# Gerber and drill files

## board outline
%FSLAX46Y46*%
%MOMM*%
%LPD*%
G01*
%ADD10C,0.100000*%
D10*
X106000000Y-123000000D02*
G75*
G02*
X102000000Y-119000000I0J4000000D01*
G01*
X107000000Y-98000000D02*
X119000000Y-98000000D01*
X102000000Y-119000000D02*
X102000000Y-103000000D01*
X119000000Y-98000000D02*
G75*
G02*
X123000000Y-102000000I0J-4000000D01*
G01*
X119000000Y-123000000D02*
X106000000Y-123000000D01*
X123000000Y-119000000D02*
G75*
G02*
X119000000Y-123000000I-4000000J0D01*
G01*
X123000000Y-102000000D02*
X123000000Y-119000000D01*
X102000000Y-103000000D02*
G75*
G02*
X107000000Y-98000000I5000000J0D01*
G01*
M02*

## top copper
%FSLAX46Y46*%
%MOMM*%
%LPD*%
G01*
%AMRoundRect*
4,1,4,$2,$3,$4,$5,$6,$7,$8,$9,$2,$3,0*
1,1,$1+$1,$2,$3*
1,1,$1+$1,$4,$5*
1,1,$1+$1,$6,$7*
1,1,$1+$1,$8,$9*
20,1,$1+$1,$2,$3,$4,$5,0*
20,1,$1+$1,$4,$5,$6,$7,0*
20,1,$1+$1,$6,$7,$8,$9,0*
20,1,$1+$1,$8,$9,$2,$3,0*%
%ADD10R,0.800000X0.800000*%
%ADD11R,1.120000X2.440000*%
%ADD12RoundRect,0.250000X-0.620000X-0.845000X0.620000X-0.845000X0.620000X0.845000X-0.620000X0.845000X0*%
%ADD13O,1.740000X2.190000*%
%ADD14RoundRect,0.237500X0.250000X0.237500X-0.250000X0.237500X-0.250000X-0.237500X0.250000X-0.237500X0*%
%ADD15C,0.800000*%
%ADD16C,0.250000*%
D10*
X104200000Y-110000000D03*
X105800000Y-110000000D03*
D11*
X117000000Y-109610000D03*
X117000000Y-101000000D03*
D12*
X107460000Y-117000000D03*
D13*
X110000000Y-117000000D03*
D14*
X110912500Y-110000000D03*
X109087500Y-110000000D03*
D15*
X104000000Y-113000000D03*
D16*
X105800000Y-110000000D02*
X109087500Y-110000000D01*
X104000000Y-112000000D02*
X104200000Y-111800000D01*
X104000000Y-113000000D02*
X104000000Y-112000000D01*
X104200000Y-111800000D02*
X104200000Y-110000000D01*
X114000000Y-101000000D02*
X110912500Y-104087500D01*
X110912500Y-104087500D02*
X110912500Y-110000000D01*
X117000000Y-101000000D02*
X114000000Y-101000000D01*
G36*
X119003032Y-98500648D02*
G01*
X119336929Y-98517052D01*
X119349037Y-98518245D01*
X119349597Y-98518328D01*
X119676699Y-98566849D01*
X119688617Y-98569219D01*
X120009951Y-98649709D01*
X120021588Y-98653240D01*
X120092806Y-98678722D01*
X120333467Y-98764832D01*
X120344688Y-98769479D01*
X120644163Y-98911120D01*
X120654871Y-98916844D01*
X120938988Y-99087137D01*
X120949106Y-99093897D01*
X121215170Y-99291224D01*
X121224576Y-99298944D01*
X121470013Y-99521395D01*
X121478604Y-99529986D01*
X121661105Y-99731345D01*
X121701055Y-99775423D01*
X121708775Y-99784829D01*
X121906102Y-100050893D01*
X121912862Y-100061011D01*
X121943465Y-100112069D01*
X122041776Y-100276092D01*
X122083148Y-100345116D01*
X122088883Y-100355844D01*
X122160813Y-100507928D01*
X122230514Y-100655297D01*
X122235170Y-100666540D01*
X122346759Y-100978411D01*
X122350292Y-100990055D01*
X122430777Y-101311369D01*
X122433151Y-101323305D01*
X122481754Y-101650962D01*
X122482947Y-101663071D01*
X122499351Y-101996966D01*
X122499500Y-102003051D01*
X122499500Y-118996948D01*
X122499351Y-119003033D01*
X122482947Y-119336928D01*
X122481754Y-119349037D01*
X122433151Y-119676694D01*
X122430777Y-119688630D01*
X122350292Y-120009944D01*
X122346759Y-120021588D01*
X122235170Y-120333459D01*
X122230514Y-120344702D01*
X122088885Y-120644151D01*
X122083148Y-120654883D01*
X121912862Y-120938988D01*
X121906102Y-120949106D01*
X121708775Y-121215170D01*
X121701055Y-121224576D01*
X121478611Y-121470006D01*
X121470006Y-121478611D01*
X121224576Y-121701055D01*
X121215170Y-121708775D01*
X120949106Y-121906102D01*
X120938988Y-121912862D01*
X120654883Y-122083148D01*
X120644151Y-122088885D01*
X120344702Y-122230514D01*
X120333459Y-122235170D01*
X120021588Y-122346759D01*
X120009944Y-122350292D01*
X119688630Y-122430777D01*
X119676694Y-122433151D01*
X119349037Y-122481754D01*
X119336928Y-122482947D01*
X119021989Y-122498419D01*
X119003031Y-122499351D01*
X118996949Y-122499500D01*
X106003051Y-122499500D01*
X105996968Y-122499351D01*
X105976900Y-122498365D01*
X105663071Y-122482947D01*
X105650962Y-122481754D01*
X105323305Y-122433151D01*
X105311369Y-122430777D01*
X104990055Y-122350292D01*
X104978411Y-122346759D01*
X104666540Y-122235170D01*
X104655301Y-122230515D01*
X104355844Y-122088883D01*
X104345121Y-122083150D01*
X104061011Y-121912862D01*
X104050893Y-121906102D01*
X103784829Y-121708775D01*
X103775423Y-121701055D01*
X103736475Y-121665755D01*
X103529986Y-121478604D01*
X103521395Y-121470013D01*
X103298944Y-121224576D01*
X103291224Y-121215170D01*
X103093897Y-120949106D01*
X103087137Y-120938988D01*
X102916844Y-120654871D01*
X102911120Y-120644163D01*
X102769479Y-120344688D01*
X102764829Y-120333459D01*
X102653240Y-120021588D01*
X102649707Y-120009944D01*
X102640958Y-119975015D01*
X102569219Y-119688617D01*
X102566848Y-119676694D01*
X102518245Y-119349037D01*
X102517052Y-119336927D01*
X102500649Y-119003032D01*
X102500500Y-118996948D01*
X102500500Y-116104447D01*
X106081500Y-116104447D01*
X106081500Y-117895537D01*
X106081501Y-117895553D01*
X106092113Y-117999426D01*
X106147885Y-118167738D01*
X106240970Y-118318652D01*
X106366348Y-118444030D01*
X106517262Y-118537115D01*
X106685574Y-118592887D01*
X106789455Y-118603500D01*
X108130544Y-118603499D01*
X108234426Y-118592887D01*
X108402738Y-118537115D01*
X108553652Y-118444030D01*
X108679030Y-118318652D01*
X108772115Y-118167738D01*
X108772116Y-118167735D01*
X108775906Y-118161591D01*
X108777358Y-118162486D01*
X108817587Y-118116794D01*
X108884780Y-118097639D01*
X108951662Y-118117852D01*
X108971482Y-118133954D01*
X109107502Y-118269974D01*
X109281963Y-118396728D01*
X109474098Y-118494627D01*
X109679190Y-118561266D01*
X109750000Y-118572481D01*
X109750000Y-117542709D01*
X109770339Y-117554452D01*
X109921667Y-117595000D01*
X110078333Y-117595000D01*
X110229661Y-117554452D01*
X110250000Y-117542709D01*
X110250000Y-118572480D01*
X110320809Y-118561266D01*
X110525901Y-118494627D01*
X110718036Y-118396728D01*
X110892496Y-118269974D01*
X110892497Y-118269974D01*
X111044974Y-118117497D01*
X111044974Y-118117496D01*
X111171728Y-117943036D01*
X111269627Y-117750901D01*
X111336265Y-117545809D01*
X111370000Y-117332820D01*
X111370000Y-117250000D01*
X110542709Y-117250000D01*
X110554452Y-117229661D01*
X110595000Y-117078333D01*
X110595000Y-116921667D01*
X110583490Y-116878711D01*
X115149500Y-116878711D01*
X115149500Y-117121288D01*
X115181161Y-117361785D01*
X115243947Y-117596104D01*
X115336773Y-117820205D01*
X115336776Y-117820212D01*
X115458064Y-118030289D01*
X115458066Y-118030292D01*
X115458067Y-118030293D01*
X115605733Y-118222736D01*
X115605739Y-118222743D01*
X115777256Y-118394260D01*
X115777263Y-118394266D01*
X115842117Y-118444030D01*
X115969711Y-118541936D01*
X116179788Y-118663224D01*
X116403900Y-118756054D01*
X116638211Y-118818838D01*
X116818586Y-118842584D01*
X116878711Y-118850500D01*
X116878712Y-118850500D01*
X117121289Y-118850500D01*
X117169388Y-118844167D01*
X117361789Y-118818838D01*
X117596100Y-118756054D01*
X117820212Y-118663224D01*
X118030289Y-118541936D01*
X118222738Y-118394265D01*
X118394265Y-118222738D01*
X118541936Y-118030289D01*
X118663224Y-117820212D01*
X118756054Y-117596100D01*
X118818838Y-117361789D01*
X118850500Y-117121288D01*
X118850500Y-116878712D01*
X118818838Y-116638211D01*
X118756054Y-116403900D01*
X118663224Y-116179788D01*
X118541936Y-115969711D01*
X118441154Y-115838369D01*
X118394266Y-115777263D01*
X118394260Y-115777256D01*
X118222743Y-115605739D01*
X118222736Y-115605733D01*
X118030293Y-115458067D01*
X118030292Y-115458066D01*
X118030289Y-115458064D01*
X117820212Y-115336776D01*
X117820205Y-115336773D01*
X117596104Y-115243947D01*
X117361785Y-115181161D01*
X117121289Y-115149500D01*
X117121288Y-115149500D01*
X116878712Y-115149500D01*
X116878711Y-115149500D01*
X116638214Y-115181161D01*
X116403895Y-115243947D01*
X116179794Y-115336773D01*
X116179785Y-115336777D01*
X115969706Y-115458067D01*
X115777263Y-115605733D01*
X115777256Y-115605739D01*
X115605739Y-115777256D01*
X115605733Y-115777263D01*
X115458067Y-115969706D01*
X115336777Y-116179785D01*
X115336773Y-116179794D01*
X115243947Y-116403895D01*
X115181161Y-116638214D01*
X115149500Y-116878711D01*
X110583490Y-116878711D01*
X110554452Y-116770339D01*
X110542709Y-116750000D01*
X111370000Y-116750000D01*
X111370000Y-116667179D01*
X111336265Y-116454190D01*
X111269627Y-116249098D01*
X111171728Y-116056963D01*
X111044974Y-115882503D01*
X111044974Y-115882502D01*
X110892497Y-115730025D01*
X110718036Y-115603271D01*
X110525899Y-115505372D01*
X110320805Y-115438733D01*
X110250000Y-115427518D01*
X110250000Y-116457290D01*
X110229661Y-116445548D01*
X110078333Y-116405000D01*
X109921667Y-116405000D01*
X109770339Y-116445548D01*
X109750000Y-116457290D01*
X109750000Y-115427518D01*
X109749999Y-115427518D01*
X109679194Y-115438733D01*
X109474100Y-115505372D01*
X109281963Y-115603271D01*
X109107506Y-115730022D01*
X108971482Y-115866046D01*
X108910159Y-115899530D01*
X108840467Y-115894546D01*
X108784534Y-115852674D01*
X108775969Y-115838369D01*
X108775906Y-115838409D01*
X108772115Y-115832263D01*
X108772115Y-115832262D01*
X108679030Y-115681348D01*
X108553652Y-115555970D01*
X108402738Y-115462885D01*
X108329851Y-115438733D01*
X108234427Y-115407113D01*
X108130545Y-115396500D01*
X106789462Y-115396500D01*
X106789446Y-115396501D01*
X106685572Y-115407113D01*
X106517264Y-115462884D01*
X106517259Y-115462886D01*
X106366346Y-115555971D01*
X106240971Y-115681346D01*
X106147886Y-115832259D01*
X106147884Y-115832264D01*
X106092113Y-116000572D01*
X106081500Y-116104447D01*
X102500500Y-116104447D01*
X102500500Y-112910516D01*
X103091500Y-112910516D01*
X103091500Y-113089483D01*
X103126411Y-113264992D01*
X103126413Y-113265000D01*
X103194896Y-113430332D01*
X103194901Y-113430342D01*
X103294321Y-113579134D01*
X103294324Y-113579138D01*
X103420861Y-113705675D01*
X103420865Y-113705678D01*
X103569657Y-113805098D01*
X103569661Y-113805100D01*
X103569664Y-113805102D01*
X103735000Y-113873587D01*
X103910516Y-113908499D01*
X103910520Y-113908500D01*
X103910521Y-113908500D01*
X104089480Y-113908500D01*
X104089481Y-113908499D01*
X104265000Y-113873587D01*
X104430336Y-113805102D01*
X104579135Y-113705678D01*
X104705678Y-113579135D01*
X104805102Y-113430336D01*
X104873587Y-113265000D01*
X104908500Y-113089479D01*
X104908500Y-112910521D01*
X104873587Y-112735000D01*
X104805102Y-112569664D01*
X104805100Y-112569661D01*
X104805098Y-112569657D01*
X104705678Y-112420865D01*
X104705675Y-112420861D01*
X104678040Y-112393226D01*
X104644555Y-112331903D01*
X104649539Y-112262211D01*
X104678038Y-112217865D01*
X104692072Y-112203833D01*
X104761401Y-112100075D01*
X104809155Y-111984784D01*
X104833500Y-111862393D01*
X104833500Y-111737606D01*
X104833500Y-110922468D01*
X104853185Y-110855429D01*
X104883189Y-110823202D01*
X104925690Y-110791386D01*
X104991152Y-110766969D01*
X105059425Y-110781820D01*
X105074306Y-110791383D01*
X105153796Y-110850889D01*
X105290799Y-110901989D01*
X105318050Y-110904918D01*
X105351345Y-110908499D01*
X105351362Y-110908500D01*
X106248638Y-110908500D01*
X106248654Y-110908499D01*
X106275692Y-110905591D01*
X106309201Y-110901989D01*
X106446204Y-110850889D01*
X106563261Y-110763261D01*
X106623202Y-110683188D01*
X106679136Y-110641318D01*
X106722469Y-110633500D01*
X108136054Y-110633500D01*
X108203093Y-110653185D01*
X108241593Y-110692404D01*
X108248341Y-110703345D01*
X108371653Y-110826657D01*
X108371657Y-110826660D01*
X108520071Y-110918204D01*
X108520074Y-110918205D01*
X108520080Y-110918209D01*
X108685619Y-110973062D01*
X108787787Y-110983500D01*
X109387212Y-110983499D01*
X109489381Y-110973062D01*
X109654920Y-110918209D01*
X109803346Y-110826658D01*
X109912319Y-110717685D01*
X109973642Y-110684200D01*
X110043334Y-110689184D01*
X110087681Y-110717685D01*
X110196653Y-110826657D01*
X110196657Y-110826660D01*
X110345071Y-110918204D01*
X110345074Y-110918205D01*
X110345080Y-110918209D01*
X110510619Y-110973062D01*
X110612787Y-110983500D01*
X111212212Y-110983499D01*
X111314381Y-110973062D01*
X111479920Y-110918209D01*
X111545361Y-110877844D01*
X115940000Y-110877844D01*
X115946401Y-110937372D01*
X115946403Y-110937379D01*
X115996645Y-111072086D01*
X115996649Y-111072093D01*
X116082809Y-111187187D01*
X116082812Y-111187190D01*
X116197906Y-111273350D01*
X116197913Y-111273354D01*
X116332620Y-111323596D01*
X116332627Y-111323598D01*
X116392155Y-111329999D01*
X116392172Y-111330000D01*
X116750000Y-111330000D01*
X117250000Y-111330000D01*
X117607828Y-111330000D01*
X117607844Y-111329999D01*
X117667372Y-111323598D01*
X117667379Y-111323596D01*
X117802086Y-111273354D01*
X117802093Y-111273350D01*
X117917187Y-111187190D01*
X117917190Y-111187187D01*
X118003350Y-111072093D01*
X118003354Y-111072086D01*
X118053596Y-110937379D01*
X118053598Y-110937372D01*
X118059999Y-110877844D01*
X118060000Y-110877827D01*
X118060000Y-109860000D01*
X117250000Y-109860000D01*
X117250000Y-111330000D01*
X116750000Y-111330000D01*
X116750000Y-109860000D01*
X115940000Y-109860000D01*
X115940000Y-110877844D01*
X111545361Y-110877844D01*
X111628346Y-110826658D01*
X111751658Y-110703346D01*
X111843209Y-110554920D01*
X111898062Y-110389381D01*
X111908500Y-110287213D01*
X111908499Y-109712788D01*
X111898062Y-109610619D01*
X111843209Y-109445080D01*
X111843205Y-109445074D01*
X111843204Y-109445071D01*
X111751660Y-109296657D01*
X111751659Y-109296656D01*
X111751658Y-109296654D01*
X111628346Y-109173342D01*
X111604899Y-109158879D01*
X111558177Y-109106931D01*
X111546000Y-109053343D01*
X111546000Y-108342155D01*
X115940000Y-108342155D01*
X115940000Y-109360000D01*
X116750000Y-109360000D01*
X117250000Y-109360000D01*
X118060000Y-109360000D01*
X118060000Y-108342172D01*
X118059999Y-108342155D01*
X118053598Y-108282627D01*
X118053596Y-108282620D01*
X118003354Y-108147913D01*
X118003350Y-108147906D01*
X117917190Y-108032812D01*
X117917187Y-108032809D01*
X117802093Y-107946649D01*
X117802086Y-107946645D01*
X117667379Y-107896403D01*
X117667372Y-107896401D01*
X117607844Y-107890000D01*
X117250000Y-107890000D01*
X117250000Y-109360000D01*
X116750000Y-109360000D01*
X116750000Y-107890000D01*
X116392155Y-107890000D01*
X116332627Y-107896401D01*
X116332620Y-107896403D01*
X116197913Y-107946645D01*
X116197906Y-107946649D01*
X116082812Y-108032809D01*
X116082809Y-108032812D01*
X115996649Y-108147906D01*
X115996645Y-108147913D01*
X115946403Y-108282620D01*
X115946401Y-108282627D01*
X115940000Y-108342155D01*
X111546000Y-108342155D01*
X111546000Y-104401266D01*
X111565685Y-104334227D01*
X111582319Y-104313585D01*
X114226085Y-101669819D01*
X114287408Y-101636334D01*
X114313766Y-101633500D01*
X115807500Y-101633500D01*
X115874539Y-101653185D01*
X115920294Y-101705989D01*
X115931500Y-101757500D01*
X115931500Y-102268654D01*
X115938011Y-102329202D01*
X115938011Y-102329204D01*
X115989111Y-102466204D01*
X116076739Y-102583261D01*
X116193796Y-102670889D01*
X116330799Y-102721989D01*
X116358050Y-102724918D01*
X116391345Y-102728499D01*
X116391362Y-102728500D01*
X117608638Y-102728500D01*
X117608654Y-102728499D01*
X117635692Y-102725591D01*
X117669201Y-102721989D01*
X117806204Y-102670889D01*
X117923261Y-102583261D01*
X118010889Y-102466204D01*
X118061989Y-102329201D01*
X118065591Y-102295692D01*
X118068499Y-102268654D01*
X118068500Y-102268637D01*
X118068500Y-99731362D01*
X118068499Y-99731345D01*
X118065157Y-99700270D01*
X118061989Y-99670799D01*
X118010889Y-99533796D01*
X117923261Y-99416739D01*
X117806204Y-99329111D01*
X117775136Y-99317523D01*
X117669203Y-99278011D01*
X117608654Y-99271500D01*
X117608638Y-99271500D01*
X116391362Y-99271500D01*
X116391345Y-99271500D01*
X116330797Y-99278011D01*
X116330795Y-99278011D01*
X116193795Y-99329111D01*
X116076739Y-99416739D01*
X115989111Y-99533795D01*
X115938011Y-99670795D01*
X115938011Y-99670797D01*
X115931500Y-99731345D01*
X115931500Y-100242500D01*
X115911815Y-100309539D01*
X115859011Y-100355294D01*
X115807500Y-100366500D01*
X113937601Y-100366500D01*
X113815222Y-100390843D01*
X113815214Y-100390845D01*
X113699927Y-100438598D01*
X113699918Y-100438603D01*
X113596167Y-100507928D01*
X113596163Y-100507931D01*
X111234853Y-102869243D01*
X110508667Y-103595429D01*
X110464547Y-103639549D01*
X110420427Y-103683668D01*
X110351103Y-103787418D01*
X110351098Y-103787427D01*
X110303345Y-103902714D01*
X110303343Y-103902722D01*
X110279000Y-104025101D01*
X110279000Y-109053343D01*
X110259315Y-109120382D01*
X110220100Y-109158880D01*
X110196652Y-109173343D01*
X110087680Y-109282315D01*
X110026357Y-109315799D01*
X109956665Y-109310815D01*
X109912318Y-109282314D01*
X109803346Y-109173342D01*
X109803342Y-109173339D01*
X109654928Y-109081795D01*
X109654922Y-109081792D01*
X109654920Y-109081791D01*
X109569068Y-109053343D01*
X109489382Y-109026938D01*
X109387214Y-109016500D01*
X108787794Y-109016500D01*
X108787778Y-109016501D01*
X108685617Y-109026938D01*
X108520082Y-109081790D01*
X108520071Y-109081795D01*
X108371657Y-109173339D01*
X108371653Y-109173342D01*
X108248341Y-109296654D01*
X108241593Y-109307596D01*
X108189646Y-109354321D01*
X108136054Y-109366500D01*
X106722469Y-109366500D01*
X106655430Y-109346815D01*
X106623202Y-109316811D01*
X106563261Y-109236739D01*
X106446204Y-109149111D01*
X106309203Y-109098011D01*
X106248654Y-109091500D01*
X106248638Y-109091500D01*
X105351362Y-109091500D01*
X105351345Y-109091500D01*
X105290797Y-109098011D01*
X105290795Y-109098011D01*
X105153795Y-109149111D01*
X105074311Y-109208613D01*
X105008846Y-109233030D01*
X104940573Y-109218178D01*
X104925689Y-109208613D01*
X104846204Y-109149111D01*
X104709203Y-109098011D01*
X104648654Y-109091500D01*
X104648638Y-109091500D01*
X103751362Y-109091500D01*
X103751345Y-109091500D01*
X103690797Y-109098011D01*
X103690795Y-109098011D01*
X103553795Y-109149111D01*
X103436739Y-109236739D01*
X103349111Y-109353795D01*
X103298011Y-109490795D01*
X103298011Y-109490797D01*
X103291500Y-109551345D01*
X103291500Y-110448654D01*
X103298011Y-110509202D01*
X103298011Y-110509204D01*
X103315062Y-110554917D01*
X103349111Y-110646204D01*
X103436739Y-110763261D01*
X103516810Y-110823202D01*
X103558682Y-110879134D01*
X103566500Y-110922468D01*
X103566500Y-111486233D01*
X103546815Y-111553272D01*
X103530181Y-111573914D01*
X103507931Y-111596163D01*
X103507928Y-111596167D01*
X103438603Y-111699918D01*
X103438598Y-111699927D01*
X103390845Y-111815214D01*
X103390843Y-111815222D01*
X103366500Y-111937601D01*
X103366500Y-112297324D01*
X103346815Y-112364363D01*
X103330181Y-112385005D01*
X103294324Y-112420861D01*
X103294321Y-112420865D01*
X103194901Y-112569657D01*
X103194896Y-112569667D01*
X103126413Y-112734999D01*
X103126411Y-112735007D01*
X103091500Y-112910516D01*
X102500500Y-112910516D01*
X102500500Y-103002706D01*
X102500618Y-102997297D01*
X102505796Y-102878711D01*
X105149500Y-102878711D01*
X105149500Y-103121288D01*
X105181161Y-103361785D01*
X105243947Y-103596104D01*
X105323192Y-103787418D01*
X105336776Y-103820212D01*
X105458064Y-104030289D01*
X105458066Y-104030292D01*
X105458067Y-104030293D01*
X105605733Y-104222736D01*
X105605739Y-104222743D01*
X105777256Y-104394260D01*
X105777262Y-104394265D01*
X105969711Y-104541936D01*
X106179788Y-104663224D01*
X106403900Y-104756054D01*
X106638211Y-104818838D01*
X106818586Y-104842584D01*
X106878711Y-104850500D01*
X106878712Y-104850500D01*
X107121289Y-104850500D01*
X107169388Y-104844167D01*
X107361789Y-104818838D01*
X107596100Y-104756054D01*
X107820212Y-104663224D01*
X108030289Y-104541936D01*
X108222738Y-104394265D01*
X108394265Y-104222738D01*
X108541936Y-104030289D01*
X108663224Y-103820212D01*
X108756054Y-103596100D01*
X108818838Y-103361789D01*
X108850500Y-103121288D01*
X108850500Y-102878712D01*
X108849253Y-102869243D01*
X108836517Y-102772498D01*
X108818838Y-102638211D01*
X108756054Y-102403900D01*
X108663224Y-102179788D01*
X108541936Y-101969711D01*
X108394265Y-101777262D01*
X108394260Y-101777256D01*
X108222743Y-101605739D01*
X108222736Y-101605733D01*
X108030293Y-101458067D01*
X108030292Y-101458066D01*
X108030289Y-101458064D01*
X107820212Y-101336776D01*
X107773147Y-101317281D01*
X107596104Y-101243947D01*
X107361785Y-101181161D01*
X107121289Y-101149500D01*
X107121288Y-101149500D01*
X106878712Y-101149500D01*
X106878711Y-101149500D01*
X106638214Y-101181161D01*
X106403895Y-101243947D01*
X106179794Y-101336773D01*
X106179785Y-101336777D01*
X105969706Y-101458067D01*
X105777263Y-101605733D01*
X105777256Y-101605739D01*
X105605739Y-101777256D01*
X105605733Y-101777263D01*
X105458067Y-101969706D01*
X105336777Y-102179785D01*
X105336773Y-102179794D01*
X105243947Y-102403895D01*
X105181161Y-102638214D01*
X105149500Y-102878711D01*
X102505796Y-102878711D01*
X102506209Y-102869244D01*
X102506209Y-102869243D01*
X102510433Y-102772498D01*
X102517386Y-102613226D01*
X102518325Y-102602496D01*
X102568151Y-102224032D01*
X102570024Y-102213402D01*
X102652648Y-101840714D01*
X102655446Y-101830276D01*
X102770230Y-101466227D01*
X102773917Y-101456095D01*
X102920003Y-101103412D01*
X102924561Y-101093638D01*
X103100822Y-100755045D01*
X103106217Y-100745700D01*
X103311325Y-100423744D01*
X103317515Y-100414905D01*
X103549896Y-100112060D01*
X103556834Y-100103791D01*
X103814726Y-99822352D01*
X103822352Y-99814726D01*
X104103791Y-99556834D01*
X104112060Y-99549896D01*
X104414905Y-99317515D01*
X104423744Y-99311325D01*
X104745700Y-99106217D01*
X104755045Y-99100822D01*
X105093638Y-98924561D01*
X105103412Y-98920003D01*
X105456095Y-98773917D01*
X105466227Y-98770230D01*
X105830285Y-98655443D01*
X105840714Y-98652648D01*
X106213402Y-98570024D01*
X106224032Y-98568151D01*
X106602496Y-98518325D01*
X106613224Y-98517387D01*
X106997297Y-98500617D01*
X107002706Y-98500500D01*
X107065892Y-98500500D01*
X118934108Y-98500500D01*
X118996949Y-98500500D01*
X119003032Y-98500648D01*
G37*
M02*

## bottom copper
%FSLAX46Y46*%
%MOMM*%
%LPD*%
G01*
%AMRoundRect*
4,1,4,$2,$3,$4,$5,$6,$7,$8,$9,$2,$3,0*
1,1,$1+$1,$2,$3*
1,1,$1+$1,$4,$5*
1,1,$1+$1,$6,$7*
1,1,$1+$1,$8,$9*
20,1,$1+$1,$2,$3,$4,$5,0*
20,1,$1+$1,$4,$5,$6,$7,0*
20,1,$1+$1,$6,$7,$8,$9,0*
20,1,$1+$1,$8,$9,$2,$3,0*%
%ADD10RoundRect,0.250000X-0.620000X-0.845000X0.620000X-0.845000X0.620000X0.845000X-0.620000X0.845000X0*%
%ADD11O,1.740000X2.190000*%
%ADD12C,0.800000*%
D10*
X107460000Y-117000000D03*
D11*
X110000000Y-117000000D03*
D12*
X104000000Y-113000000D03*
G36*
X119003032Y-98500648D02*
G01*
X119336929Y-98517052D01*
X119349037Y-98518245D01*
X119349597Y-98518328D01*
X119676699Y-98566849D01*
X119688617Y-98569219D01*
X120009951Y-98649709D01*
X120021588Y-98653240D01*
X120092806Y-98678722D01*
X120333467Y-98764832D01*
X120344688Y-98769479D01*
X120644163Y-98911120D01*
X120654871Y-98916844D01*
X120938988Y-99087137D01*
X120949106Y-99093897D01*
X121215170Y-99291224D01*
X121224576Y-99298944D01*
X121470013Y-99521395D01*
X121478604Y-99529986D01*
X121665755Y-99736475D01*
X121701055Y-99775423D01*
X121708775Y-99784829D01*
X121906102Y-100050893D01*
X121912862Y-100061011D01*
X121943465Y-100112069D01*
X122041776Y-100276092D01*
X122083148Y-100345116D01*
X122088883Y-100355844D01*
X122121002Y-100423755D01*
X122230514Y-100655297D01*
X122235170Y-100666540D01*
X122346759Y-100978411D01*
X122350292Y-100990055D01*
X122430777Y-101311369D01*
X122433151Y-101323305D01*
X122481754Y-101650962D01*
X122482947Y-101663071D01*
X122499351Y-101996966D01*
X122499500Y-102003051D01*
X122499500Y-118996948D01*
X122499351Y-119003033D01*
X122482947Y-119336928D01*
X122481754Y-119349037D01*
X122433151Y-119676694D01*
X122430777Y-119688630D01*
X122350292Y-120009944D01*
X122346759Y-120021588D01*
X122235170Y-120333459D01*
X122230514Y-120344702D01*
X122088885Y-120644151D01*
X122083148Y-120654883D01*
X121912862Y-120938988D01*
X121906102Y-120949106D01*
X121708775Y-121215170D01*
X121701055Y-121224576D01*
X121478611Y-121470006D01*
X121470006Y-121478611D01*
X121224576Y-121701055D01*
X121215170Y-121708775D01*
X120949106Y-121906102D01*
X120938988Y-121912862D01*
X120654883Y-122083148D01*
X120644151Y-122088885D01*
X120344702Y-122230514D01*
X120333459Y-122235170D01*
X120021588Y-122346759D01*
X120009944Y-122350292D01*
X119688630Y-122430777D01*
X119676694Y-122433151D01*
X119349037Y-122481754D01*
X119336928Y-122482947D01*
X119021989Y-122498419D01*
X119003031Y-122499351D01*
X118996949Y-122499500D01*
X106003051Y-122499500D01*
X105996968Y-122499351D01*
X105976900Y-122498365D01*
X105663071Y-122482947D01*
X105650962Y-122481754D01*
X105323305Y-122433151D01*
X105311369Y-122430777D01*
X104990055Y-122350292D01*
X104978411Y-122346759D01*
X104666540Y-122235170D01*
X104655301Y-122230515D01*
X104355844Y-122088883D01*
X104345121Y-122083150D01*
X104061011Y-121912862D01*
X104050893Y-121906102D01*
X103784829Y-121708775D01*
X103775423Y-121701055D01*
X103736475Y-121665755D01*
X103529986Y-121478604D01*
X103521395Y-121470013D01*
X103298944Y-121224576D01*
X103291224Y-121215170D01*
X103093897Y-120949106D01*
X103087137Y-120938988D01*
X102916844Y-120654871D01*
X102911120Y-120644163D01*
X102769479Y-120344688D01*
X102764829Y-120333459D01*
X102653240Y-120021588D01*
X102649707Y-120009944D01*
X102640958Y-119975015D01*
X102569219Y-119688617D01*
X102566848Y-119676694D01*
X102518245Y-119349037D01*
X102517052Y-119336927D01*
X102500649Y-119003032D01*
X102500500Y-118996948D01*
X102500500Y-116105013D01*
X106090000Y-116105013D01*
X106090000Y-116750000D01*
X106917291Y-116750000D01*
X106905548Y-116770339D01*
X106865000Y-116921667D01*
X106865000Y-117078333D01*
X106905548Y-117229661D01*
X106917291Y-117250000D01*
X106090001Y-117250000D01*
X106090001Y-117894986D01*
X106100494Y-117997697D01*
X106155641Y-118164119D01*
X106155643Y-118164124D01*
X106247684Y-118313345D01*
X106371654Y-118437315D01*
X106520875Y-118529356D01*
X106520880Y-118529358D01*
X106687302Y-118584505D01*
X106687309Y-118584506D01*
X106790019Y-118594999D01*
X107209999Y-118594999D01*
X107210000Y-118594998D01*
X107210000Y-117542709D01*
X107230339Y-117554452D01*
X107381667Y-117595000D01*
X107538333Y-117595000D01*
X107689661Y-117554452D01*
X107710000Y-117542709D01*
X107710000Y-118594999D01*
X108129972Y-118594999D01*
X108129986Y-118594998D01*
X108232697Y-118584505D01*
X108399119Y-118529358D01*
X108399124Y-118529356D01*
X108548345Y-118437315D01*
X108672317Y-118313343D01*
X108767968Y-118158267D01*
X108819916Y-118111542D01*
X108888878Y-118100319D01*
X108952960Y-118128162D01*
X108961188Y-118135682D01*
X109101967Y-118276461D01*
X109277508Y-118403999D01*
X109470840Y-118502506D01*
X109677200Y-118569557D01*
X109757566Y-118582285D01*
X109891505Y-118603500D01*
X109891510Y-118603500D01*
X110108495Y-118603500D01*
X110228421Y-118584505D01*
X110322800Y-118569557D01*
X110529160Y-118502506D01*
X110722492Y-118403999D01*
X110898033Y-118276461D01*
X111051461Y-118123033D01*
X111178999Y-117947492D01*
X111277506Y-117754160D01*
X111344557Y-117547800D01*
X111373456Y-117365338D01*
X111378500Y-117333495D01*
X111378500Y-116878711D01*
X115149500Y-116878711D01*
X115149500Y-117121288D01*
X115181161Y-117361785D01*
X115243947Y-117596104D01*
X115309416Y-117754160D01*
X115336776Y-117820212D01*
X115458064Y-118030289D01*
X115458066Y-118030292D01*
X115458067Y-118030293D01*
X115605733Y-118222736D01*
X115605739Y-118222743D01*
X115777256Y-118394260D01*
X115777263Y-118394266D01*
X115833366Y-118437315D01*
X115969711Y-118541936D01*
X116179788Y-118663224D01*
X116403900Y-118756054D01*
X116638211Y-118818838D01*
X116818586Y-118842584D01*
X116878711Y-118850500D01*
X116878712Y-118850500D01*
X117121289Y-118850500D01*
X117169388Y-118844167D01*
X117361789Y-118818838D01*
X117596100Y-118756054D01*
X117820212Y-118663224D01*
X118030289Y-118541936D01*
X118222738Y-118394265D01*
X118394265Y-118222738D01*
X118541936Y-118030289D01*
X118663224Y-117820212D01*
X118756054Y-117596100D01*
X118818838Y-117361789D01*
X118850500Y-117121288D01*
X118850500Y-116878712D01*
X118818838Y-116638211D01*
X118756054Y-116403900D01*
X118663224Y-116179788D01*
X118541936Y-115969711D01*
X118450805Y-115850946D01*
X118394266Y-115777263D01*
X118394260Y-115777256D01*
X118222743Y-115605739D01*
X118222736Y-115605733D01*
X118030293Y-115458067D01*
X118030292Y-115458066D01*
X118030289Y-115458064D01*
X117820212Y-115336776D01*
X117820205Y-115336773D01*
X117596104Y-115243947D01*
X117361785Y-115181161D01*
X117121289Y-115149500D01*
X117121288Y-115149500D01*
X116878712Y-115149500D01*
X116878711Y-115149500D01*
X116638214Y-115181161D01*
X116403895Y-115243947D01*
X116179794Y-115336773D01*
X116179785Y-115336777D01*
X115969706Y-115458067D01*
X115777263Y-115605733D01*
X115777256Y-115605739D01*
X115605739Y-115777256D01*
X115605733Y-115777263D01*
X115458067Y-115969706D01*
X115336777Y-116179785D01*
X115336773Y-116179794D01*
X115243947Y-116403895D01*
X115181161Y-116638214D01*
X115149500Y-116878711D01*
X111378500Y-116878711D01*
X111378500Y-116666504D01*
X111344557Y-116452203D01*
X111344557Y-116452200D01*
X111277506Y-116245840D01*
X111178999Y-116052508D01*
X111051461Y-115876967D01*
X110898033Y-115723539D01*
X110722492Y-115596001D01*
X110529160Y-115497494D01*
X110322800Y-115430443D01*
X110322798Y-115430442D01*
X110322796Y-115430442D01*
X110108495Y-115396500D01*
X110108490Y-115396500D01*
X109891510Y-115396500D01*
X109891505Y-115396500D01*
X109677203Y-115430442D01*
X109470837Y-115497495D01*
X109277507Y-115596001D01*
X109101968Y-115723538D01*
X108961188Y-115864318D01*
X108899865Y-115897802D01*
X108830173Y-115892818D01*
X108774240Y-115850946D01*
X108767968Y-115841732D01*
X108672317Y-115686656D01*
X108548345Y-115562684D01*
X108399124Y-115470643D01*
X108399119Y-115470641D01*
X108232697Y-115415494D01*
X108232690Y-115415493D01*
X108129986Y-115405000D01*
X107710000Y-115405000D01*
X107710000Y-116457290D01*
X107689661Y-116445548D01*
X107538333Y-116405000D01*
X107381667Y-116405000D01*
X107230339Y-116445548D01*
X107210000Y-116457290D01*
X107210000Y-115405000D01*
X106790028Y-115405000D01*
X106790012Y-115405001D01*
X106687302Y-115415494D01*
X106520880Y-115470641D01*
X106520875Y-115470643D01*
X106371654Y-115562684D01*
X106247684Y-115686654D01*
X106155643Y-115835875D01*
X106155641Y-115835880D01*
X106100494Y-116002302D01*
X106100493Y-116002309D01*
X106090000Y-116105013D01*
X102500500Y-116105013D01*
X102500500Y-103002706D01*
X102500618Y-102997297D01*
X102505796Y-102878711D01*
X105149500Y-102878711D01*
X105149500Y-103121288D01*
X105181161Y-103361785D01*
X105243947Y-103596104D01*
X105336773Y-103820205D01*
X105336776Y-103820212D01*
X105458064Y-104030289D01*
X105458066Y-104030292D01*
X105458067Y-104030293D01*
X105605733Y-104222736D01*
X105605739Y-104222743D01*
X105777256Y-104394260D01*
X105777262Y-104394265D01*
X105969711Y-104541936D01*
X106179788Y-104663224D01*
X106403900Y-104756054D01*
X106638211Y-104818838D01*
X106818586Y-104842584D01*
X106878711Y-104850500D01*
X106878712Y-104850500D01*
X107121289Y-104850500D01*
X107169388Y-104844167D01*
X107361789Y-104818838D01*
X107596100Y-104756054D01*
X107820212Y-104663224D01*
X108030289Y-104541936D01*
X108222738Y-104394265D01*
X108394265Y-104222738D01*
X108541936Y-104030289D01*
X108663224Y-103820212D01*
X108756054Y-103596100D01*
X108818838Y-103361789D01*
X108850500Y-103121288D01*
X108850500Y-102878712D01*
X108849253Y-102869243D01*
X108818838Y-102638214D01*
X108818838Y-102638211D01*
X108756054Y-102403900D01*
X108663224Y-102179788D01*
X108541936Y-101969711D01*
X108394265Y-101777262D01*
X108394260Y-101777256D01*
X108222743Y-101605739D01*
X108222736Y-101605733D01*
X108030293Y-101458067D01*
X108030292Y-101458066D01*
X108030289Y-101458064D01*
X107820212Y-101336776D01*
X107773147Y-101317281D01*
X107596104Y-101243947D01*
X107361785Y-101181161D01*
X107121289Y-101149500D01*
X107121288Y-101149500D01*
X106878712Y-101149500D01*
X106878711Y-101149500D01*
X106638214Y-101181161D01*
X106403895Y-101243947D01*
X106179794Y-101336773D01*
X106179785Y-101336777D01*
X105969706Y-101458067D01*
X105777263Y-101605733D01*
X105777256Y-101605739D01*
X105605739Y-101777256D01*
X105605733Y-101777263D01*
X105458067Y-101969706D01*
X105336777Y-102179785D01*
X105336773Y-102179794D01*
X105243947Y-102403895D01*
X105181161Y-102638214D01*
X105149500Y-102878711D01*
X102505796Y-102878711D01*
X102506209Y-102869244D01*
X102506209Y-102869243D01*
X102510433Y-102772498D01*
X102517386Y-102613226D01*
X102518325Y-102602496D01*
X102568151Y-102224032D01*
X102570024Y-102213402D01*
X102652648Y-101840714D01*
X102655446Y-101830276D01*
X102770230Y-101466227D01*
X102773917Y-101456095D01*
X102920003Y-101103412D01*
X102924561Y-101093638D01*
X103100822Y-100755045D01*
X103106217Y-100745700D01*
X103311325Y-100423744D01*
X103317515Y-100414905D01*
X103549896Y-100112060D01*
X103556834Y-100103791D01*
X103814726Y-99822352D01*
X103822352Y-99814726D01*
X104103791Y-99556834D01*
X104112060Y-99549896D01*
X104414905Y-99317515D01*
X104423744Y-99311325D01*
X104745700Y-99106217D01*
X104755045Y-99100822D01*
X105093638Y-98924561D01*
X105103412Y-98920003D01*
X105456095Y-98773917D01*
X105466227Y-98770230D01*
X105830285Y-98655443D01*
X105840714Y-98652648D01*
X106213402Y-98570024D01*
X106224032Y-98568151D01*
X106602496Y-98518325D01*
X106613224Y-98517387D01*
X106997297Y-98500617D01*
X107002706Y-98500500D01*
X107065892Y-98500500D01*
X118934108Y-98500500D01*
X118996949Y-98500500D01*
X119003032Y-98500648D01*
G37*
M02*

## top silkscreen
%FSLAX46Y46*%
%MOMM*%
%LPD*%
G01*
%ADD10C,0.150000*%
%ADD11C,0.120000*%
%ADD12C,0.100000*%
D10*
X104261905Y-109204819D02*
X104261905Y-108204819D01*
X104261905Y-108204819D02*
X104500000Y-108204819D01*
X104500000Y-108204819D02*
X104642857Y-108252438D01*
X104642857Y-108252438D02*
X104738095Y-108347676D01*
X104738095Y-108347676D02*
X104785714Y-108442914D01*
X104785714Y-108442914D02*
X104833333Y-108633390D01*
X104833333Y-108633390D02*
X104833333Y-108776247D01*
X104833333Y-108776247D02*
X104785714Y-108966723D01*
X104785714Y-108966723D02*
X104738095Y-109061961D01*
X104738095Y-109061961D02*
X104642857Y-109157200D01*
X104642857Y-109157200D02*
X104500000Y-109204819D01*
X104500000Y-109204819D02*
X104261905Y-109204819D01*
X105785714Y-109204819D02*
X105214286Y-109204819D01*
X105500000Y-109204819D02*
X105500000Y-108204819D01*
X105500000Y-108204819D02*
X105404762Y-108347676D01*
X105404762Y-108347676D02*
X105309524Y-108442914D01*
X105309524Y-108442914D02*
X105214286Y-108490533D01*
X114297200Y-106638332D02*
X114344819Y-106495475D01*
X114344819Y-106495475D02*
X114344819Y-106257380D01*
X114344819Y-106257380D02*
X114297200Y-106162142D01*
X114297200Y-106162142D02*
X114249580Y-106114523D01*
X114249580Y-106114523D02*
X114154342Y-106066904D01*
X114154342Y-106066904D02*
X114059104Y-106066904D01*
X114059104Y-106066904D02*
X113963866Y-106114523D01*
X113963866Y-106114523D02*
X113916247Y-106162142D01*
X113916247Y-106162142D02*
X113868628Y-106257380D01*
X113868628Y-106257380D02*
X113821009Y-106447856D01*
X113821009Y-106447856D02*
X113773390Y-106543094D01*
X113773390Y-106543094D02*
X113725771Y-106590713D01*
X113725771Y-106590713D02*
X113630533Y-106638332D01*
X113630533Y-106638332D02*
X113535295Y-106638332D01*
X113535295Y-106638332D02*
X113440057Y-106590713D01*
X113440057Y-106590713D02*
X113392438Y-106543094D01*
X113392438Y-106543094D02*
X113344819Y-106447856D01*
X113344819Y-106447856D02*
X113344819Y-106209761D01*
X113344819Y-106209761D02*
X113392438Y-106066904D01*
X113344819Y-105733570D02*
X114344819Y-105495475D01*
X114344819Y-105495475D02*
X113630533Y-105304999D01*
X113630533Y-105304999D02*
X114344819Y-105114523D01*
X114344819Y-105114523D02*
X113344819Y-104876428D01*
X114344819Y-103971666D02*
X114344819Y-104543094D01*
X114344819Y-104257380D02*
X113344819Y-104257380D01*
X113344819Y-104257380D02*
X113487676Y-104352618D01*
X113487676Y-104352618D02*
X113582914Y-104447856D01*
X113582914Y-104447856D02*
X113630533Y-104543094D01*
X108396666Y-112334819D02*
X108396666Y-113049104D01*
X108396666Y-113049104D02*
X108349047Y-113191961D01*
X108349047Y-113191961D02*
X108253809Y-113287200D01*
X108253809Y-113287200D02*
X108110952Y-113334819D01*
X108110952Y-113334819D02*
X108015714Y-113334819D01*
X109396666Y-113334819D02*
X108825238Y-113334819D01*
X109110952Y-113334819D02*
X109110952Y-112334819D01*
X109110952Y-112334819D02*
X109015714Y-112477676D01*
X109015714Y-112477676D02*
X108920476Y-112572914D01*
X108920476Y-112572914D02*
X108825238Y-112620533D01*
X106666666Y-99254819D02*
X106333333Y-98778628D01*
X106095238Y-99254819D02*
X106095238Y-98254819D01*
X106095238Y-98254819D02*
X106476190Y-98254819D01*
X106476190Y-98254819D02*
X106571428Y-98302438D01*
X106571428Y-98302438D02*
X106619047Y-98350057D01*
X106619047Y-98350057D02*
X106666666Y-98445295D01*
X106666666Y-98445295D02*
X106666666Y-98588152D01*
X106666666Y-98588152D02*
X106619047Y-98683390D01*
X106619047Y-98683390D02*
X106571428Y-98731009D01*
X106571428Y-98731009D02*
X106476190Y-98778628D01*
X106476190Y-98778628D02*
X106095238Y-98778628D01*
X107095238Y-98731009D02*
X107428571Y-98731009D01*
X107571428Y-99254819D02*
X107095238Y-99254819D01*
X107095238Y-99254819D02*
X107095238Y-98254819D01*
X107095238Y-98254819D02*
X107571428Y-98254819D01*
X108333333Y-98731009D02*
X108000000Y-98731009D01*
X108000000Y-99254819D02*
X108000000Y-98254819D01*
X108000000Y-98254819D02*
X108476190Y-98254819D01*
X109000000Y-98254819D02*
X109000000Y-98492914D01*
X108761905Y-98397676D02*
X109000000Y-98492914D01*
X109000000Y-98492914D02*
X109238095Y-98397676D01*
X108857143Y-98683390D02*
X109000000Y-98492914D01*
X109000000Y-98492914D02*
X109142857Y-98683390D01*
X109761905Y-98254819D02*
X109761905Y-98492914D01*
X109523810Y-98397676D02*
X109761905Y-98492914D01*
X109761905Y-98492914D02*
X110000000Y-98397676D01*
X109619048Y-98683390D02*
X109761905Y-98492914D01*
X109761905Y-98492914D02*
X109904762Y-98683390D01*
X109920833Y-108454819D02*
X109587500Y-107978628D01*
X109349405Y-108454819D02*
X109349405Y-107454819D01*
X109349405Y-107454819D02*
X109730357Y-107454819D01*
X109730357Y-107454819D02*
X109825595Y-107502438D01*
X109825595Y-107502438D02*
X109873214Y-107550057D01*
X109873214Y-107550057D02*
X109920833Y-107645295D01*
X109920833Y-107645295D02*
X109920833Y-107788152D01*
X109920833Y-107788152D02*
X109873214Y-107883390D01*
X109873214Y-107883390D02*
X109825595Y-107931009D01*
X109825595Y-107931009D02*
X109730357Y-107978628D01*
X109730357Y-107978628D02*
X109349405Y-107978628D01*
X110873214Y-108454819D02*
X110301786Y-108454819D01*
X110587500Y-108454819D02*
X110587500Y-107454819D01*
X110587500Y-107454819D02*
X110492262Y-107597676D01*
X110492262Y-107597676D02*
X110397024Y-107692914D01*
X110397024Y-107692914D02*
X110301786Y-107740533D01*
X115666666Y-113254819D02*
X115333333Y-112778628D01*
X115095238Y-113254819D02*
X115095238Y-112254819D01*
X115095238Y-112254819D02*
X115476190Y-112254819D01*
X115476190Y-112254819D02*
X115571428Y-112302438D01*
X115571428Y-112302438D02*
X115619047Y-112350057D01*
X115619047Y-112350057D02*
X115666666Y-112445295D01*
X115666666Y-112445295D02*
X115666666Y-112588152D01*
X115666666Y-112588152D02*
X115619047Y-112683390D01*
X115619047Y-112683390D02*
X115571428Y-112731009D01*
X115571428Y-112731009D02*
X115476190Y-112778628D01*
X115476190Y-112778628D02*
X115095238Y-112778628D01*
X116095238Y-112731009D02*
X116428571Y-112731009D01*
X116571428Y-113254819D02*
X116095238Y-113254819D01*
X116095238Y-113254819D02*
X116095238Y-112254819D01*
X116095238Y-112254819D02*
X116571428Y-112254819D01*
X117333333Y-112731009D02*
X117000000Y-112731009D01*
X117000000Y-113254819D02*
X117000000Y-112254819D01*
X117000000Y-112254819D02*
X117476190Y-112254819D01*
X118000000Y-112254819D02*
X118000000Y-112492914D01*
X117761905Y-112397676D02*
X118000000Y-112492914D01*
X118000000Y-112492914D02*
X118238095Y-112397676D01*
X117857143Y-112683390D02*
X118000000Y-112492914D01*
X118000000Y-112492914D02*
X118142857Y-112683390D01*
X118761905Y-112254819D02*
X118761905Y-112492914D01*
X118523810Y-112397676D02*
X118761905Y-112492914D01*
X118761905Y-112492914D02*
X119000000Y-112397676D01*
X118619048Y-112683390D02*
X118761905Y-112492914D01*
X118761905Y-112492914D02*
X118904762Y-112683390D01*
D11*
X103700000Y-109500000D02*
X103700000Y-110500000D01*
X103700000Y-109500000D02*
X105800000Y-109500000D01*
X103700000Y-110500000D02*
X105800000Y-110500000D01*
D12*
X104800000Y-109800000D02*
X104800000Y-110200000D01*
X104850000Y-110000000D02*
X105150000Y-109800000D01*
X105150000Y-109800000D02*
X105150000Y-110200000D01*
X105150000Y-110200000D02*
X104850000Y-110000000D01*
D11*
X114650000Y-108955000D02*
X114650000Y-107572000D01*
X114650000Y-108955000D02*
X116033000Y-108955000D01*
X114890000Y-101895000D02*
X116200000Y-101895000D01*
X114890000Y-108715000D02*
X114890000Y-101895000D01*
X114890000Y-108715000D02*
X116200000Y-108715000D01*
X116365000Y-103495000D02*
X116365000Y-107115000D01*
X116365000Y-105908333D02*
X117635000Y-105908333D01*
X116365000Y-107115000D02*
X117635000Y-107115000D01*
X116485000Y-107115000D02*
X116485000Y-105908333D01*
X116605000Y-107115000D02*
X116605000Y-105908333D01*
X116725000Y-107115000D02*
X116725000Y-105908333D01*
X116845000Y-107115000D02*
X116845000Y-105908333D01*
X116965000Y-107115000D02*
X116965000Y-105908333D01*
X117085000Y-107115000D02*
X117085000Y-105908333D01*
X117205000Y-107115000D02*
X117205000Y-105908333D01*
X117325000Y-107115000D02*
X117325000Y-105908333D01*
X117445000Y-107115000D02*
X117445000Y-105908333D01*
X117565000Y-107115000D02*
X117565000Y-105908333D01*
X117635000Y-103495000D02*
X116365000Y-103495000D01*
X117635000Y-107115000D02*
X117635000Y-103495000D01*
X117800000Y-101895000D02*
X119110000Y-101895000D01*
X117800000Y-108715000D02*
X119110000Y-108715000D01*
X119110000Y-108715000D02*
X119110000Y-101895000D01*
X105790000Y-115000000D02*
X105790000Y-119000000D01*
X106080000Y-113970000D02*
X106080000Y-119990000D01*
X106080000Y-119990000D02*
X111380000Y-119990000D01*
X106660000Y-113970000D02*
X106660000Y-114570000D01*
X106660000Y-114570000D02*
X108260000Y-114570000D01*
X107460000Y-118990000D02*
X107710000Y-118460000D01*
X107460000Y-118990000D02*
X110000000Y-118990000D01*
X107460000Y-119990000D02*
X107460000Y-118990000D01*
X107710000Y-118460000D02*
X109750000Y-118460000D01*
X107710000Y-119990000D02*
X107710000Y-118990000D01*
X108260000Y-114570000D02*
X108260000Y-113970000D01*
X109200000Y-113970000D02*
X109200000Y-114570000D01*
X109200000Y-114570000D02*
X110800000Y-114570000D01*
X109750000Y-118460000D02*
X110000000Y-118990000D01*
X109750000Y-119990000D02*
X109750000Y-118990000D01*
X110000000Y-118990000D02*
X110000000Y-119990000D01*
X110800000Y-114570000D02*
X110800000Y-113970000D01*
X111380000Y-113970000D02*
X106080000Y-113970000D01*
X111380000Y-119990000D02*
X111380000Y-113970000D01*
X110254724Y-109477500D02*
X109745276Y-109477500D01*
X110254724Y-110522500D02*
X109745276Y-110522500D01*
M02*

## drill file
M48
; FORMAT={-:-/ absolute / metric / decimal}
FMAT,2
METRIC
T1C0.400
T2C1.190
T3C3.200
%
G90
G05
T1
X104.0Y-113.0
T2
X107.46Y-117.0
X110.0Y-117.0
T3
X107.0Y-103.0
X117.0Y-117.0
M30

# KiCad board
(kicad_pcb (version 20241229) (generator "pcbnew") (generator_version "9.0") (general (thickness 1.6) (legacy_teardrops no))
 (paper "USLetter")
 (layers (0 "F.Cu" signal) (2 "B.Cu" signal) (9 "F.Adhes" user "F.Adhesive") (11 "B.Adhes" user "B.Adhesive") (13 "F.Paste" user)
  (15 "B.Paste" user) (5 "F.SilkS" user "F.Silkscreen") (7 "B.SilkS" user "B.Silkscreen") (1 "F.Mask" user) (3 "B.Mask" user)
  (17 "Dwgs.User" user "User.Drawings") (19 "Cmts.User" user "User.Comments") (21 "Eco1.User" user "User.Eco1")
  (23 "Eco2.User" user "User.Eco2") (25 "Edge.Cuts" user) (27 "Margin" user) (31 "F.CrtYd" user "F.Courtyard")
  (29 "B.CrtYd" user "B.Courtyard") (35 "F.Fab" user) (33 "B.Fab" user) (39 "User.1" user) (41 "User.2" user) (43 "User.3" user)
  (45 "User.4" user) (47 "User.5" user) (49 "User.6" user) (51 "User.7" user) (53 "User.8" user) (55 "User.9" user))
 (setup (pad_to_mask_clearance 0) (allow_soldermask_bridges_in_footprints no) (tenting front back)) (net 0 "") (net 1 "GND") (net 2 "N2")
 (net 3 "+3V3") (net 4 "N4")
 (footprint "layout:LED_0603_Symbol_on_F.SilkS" (layer "F.Cu") (at 105 110)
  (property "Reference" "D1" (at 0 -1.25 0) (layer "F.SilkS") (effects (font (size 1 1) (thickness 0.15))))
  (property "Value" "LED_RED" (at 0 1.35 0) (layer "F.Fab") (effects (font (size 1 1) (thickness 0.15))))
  (fp_line (start -1.3 -0.5) (end -1.3 0.5) (stroke (width 0.12) (type solid)) (layer "F.SilkS"))
  (fp_line (start -1.3 -0.5) (end 0.8 -0.5) (stroke (width 0.12) (type solid)) (layer "F.SilkS"))
  (fp_line (start -1.3 0.5) (end 0.8 0.5) (stroke (width 0.12) (type solid)) (layer "F.SilkS"))
  (fp_line (start -0.2 -0.2) (end -0.2 0.2) (stroke (width 0.1) (type solid)) (layer "F.SilkS"))
  (fp_line (start -0.15 0) (end 0.15 -0.2) (stroke (width 0.1) (type solid)) (layer "F.SilkS"))
  (fp_line (start 0.15 -0.2) (end 0.15 0.2) (stroke (width 0.1) (type solid)) (layer "F.SilkS"))
  (fp_line (start 0.15 0.2) (end -0.15 0) (stroke (width 0.1) (type solid)) (layer "F.SilkS"))
  (pad "1" smd rect (at -0.8 0 180) (size 0.8 0.8) (layers "F.Cu" "F.Mask" "F.Paste") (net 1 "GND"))
  (pad "2" smd rect (at 0.8 0 180) (size 0.8 0.8) (layers "F.Cu" "F.Mask" "F.Paste") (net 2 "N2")))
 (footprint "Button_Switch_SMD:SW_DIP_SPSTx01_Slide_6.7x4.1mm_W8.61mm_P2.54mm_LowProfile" (layer "F.Cu") (at 117 105.305 90)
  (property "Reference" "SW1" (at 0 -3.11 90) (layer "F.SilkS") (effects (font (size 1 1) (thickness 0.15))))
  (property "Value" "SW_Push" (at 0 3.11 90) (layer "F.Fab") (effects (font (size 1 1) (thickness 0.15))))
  (fp_line (start -3.65 -2.35) (end -2.267 -2.35) (stroke (width 0.12) (type solid)) (layer "F.SilkS"))
  (fp_line (start -3.65 -2.35) (end -3.65 -0.967) (stroke (width 0.12) (type solid)) (layer "F.SilkS"))
  (fp_line (start 3.41 -2.11) (end 3.41 -0.8) (stroke (width 0.12) (type solid)) (layer "F.SilkS"))
  (fp_line (start -3.41 -2.11) (end 3.41 -2.11) (stroke (width 0.12) (type solid)) (layer "F.SilkS"))
  (fp_line (start -3.41 -2.11) (end -3.41 -0.8) (stroke (width 0.12) (type solid)) (layer "F.SilkS"))
  (fp_line (start 1.81 -0.635) (end -1.81 -0.635) (stroke (width 0.12) (type solid)) (layer "F.SilkS"))
  (fp_line (start -0.603333 -0.635) (end -0.603333 0.635) (stroke (width 0.12) (type solid)) (layer "F.SilkS"))
  (fp_line (start -1.81 -0.635) (end -1.81 0.635) (stroke (width 0.12) (type solid)) (layer "F.SilkS"))
  (fp_line (start -1.81 -0.515) (end -0.603333 -0.515) (stroke (width 0.12) (type solid)) (layer "F.SilkS"))
  (fp_line (start -1.81 -0.395) (end -0.603333 -0.395) (stroke (width 0.12) (type solid)) (layer "F.SilkS"))
  (fp_line (start -1.81 -0.275) (end -0.603333 -0.275) (stroke (width 0.12) (type solid)) (layer "F.SilkS"))
  (fp_line (start -1.81 -0.155) (end -0.603333 -0.155) (stroke (width 0.12) (type solid)) (layer "F.SilkS"))
  (fp_line (start -1.81 -0.035) (end -0.603333 -0.035) (stroke (width 0.12) (type solid)) (layer "F.SilkS"))
  (fp_line (start -1.81 0.085) (end -0.603333 0.085) (stroke (width 0.12) (type solid)) (layer "F.SilkS"))
  (fp_line (start -1.81 0.205) (end -0.603333 0.205) (stroke (width 0.12) (type solid)) (layer "F.SilkS"))
  (fp_line (start -1.81 0.325) (end -0.603333 0.325) (stroke (width 0.12) (type solid)) (layer "F.SilkS"))
  (fp_line (start -1.81 0.445) (end -0.603333 0.445) (stroke (width 0.12) (type solid)) (layer "F.SilkS"))
  (fp_line (start -1.81 0.565) (end -0.603333 0.565) (stroke (width 0.12) (type solid)) (layer "F.SilkS"))
  (fp_line (start 1.81 0.635) (end 1.81 -0.635) (stroke (width 0.12) (type solid)) (layer "F.SilkS"))
  (fp_line (start -1.81 0.635) (end 1.81 0.635) (stroke (width 0.12) (type solid)) (layer "F.SilkS"))
  (fp_line (start 3.41 0.8) (end 3.41 2.11) (stroke (width 0.12) (type solid)) (layer "F.SilkS"))
  (fp_line (start -3.41 0.8) (end -3.41 2.11) (stroke (width 0.12) (type solid)) (layer "F.SilkS"))
  (fp_line (start -3.41 2.11) (end 3.41 2.11) (stroke (width 0.12) (type solid)) (layer "F.SilkS"))
  (pad "1" smd rect (at -4.305 0 90) (size 2.44 1.12) (layers "F.Cu" "F.Mask" "F.Paste") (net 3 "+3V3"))
  (pad "2" smd rect (at 4.305 0 90) (size 2.44 1.12) (layers "F.Cu" "F.Mask" "F.Paste") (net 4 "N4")))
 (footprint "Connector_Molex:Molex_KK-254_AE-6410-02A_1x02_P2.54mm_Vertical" (layer "F.Cu") (at 107.46 117)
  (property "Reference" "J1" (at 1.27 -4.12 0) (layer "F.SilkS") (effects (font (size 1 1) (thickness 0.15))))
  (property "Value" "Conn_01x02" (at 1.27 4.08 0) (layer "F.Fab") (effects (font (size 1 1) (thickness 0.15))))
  (fp_line (start -1.67 -2) (end -1.67 2) (stroke (width 0.12) (type solid)) (layer "F.SilkS"))
  (fp_line (start -1.38 -3.03) (end -1.38 2.99) (stroke (width 0.12) (type solid)) (layer "F.SilkS"))
  (fp_line (start -1.38 2.99) (end 3.92 2.99) (stroke (width 0.12) (type solid)) (layer "F.SilkS"))
  (fp_line (start -0.8 -3.03) (end -0.8 -2.43) (stroke (width 0.12) (type solid)) (layer "F.SilkS"))
  (fp_line (start -0.8 -2.43) (end 0.8 -2.43) (stroke (width 0.12) (type solid)) (layer "F.SilkS"))
  (fp_line (start 0 1.99) (end 0.25 1.46) (stroke (width 0.12) (type solid)) (layer "F.SilkS"))
  (fp_line (start 0 1.99) (end 2.54 1.99) (stroke (width 0.12) (type solid)) (layer "F.SilkS"))
  (fp_line (start 0 2.99) (end 0 1.99) (stroke (width 0.12) (type solid)) (layer "F.SilkS"))
  (fp_line (start 0.25 1.46) (end 2.29 1.46) (stroke (width 0.12) (type solid)) (layer "F.SilkS"))
  (fp_line (start 0.25 2.99) (end 0.25 1.99) (stroke (width 0.12) (type solid)) (layer "F.SilkS"))
  (fp_line (start 0.8 -2.43) (end 0.8 -3.03) (stroke (width 0.12) (type solid)) (layer "F.SilkS"))
  (fp_line (start 1.74 -3.03) (end 1.74 -2.43) (stroke (width 0.12) (type solid)) (layer "F.SilkS"))
  (fp_line (start 1.74 -2.43) (end 3.34 -2.43) (stroke (width 0.12) (type solid)) (layer "F.SilkS"))
  (fp_line (start 2.29 1.46) (end 2.54 1.99) (stroke (width 0.12) (type solid)) (layer "F.SilkS"))
  (fp_line (start 2.29 2.99) (end 2.29 1.99) (stroke (width 0.12) (type solid)) (layer "F.SilkS"))
  (fp_line (start 2.54 1.99) (end 2.54 2.99) (stroke (width 0.12) (type solid)) (layer "F.SilkS"))
  (fp_line (start 3.34 -2.43) (end 3.34 -3.03) (stroke (width 0.12) (type solid)) (layer "F.SilkS"))
  (fp_line (start 3.92 -3.03) (end -1.38 -3.03) (stroke (width 0.12) (type solid)) (layer "F.SilkS"))
  (fp_line (start 3.92 2.99) (end 3.92 -3.03) (stroke (width 0.12) (type solid)) (layer "F.SilkS"))
  (pad "1" thru_hole roundrect (at 0 0) (size 1.74 2.19) (drill 1.19) (layers "*.Cu" "*.Mask") (remove_unused_layers no)
   (roundrect_rratio 0.143678) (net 1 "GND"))
  (pad "2" thru_hole oval (at 2.54 0) (size 1.74 2.19) (drill 1.19) (layers "*.Cu" "*.Mask") (remove_unused_layers no) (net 3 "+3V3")))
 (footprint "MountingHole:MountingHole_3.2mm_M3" (layer "F.Cu") (at 107 103)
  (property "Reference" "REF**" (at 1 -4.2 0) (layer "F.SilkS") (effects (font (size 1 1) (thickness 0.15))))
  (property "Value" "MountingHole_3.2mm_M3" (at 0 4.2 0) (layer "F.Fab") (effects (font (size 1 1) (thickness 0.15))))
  (pad "" np_thru_hole circle (at 0 0) (size 3.2 3.2) (drill 3.2) (layers "*.Cu" "*.Mask")))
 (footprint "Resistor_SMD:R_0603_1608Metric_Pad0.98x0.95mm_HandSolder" (layer "F.Cu") (at 110 110 180)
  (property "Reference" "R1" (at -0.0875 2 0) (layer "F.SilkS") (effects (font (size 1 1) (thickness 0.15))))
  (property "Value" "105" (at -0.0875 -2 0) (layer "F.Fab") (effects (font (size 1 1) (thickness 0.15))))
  (fp_line (start -0.254724 0.5225) (end 0.254724 0.5225) (stroke (width 0.12) (type solid)) (layer "F.SilkS"))
  (fp_line (start -0.254724 -0.5225) (end 0.254724 -0.5225) (stroke (width 0.12) (type solid)) (layer "F.SilkS"))
  (pad "1" smd roundrect (at -0.9125 0 180) (size 0.975 0.95) (layers "F.Cu" "F.Mask" "F.Paste") (roundrect_rratio 0.25) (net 4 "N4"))
  (pad "2" smd roundrect (at 0.9125 0 180) (size 0.975 0.95) (layers "F.Cu" "F.Mask" "F.Paste") (roundrect_rratio 0.25) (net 2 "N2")))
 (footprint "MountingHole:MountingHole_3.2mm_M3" (layer "F.Cu") (at 117 117)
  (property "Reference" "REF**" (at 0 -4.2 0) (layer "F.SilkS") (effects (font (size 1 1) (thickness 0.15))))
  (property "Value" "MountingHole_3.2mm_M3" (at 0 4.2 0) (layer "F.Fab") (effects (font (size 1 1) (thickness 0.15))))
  (pad "" np_thru_hole circle (at 0 0) (size 3.2 3.2) (drill 3.2) (layers "*.Cu" "*.Mask")))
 (gr_arc (start 106 123) (mid 103.171573 121.828427) (end 102 119) (stroke (width 0.1) (type default)) (layer "Edge.Cuts"))
 (gr_line (start 107 98) (end 119 98) (stroke (width 0.1) (type default)) (layer "Edge.Cuts"))
 (gr_line (start 102 119) (end 102 103) (stroke (width 0.1) (type default)) (layer "Edge.Cuts"))
 (gr_arc (start 119 98) (mid 121.828427 99.171573) (end 123 102) (stroke (width 0.1) (type default)) (layer "Edge.Cuts"))
 (gr_line (start 119 123) (end 106 123) (stroke (width 0.1) (type default)) (layer "Edge.Cuts"))
 (gr_arc (start 123 119) (mid 121.828427 121.828427) (end 119 123) (stroke (width 0.1) (type default)) (layer "Edge.Cuts"))
 (gr_line (start 123 102) (end 123 119) (stroke (width 0.1) (type default)) (layer "Edge.Cuts"))
 (gr_arc (start 102 103) (mid 103.464466 99.464466) (end 107 98) (stroke (width 0.1) (type default)) (layer "Edge.Cuts"))
 (segment (start 105.8 110) (end 109.0875 110) (width 0.25) (layer "F.Cu") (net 2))
 (segment (start 104 112) (end 104.2 111.8) (width 0.25) (layer "F.Cu") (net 1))
 (segment (start 104 113) (end 104 112) (width 0.25) (layer "F.Cu") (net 1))
 (segment (start 104.2 111.8) (end 104.2 110) (width 0.25) (layer "F.Cu") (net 1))
 (via (at 104 113) (size 0.8) (drill 0.4) (layers "F.Cu" "B.Cu") (free yes) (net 1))
 (segment (start 114 101) (end 110.9125 104.0875) (width 0.25) (layer "F.Cu") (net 4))
 (segment (start 110.9125 104.0875) (end 110.9125 110) (width 0.25) (layer "F.Cu") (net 4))
 (segment (start 117 101) (end 114 101) (width 0.25) (layer "F.Cu") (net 4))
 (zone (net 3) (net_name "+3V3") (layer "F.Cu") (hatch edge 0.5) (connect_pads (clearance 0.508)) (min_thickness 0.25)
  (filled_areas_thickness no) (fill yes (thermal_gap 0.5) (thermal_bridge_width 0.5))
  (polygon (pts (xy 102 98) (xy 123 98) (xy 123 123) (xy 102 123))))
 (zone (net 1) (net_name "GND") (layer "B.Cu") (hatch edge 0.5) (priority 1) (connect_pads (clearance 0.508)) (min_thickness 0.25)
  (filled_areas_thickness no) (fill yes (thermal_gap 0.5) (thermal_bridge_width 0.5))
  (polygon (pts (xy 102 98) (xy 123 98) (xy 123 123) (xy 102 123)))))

